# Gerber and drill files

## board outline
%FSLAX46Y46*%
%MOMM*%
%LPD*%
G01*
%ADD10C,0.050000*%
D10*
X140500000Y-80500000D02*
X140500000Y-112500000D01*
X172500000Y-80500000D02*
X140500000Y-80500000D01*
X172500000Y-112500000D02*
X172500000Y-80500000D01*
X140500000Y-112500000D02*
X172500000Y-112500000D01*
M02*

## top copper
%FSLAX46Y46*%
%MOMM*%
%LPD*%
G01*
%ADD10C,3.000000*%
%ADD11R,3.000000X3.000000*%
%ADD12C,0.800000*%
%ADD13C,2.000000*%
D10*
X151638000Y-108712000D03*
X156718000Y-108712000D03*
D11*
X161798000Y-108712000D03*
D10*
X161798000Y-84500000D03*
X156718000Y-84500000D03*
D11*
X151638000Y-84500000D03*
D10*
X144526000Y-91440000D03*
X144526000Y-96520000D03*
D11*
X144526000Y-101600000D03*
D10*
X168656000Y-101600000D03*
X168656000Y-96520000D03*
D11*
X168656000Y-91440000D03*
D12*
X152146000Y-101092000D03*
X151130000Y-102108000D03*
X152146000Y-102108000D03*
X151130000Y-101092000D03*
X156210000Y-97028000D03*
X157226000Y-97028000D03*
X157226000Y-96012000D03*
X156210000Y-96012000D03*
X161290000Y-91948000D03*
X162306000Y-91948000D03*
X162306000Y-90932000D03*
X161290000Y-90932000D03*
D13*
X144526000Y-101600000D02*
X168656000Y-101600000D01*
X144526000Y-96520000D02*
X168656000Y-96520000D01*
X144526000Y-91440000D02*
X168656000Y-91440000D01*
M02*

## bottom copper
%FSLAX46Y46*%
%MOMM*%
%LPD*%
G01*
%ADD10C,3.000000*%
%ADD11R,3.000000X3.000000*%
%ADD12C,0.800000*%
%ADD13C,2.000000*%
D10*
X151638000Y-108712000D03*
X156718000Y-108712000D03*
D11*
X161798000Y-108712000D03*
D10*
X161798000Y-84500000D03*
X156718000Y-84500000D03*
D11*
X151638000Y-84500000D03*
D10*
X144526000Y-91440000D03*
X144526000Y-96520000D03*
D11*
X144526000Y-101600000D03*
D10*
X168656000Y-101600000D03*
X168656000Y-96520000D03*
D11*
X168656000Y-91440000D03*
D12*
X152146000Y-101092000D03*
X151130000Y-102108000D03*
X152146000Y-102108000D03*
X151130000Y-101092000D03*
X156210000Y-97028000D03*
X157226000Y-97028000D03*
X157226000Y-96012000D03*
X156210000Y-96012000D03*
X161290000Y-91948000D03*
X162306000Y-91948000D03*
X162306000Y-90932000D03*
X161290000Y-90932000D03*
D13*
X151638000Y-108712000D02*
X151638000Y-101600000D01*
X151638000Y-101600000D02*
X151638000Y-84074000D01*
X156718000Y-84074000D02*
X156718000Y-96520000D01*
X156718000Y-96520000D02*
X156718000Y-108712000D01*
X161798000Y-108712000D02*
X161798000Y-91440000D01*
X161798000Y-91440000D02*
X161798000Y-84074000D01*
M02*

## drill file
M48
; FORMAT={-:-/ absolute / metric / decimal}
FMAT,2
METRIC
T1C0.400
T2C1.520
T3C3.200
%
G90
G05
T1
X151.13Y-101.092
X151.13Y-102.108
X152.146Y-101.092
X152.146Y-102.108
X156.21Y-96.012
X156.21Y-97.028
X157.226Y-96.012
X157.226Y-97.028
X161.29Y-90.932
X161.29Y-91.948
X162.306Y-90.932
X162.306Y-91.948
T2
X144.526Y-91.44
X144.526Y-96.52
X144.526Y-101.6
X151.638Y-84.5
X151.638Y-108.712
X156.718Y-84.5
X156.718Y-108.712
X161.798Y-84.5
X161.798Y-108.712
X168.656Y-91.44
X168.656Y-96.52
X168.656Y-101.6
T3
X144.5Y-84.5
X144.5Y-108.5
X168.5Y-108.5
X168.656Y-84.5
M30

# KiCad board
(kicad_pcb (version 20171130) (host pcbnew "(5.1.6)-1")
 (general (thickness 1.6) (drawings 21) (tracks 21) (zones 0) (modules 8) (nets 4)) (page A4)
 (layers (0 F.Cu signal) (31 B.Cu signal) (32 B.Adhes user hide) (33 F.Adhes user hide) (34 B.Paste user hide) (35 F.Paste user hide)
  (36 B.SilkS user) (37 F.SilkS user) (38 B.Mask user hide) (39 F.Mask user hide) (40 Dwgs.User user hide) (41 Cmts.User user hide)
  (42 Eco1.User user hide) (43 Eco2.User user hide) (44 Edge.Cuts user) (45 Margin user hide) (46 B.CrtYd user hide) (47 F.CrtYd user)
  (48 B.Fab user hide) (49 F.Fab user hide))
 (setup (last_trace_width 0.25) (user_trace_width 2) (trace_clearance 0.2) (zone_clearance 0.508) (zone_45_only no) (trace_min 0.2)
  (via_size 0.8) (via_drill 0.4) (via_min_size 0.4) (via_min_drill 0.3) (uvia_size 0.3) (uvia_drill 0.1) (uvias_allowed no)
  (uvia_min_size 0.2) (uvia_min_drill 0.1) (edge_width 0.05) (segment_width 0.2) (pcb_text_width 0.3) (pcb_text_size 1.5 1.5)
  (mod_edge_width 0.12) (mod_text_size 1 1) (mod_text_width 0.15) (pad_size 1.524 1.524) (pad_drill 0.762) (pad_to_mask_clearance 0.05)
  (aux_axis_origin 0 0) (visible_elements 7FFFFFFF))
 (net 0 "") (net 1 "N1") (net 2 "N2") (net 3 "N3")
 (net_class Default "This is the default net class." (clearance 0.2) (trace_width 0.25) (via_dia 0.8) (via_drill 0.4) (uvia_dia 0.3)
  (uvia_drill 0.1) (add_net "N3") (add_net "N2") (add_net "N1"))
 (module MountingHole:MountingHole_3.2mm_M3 (layer F.Cu) (at 168.5 108.5)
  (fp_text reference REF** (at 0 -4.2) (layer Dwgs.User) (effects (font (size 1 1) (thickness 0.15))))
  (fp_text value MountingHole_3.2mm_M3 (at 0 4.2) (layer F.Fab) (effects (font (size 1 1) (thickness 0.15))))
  (pad 1 np_thru_hole circle (at 0 0) (size 3.2 3.2) (drill 3.2) (layers *.Cu *.Mask)))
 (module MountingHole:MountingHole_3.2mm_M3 (layer F.Cu) (at 144.5 108.5)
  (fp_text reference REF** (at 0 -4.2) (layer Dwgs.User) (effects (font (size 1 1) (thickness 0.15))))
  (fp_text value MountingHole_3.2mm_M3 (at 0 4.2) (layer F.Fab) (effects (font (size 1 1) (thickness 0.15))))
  (pad 1 np_thru_hole circle (at 0 0) (size 3.2 3.2) (drill 3.2) (layers *.Cu *.Mask)))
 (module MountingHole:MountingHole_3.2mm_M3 (layer F.Cu) (at 144.5 84.5)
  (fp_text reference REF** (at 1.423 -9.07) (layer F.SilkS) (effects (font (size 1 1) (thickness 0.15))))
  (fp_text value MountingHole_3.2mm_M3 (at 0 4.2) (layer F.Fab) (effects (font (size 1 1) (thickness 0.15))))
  (pad 1 np_thru_hole circle (at 0 0) (size 3.2 3.2) (drill 3.2) (layers *.Cu *.Mask)))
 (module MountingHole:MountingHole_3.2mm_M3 (layer F.Cu) (at 168.656 84.5)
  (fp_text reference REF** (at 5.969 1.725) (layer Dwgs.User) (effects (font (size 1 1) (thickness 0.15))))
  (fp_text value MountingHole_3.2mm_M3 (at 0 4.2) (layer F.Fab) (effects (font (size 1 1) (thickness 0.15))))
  (pad 1 np_thru_hole circle (at 0 0) (size 3.2 3.2) (drill 3.2) (layers *.Cu *.Mask)))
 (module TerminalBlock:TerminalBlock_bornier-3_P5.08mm (layer F.Cu) (at 161.798 108.712 180)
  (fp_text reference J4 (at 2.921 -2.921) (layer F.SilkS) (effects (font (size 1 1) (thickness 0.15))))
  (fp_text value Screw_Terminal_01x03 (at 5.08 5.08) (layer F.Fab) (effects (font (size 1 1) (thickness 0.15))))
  (pad 3 thru_hole circle (at 10.16 0 180) (size 3 3) (drill 1.52) (layers *.Cu *.Mask) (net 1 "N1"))
  (pad 2 thru_hole circle (at 5.08 0 180) (size 3 3) (drill 1.52) (layers *.Cu *.Mask) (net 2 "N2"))
  (pad 1 thru_hole rect (at 0 0 180) (size 3 3) (drill 1.52) (layers *.Cu *.Mask) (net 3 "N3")))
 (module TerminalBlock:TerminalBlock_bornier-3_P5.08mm (layer F.Cu) (at 151.638 84.5)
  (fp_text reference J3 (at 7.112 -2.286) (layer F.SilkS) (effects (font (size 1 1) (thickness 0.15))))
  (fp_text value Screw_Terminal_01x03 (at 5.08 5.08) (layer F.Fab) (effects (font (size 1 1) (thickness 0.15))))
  (pad 3 thru_hole circle (at 10.16 0) (size 3 3) (drill 1.52) (layers *.Cu *.Mask) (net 3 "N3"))
  (pad 2 thru_hole circle (at 5.08 0) (size 3 3) (drill 1.52) (layers *.Cu *.Mask) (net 2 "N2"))
  (pad 1 thru_hole rect (at 0 0) (size 3 3) (drill 1.52) (layers *.Cu *.Mask) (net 1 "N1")))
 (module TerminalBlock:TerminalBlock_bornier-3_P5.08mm (layer F.Cu) (at 144.526 101.6 90)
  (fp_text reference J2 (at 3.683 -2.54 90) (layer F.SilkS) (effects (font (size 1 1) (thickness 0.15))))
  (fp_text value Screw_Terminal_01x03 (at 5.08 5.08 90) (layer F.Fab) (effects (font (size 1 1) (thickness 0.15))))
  (pad 3 thru_hole circle (at 10.16 0 90) (size 3 3) (drill 1.52) (layers *.Cu *.Mask) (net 3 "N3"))
  (pad 2 thru_hole circle (at 5.08 0 90) (size 3 3) (drill 1.52) (layers *.Cu *.Mask) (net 2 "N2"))
  (pad 1 thru_hole rect (at 0 0 90) (size 3 3) (drill 1.52) (layers *.Cu *.Mask) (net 1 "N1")))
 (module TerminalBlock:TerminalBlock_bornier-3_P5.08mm (layer F.Cu) (at 168.656 91.44 270)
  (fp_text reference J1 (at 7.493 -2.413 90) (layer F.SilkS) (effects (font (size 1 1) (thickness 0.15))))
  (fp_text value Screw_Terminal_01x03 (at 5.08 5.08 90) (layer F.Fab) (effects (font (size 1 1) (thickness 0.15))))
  (pad 3 thru_hole circle (at 10.16 0 270) (size 3 3) (drill 1.52) (layers *.Cu *.Mask) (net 1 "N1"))
  (pad 2 thru_hole circle (at 5.08 0 270) (size 3 3) (drill 1.52) (layers *.Cu *.Mask) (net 2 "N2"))
  (pad 1 thru_hole rect (at 0 0 270) (size 3 3) (drill 1.52) (layers *.Cu *.Mask) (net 3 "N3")))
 (gr_line (start 140.5 80.5) (end 140.5 112.5) (layer Edge.Cuts) (width 0.05))
 (gr_line (start 172.5 80.5) (end 140.5 80.5) (layer Edge.Cuts) (width 0.05))
 (gr_line (start 172.5 112.5) (end 172.5 80.5) (layer Edge.Cuts) (width 0.05))
 (gr_line (start 140.5 112.5) (end 172.5 112.5) (layer Edge.Cuts) (width 0.05))
 (via (at 152.146 101.092) (size 0.8) (drill 0.4) (layers F.Cu B.Cu) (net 1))
 (via (at 151.13 102.108) (size 0.8) (drill 0.4) (layers F.Cu B.Cu) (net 1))
 (via (at 152.146 102.108) (size 0.8) (drill 0.4) (layers F.Cu B.Cu) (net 1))
 (segment (start 144.526 101.6) (end 168.656 101.6) (width 2) (layer F.Cu) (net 1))
 (segment (start 151.638 108.712) (end 151.638 101.6) (width 2) (layer B.Cu) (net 1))
 (segment (start 151.638 101.6) (end 151.638 84.074) (width 2) (layer B.Cu) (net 1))
 (via (at 151.13 101.092) (size 0.8) (drill 0.4) (layers F.Cu B.Cu) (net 1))
 (via (at 156.21 97.028) (size 0.8) (drill 0.4) (layers F.Cu B.Cu) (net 2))
 (via (at 157.226 97.028) (size 0.8) (drill 0.4) (layers F.Cu B.Cu) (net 2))
 (via (at 157.226 96.012) (size 0.8) (drill 0.4) (layers F.Cu B.Cu) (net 2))
 (segment (start 144.526 96.52) (end 168.656 96.52) (width 2) (layer F.Cu) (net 2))
 (segment (start 156.718 84.074) (end 156.718 96.52) (width 2) (layer B.Cu) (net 2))
 (segment (start 156.718 96.52) (end 156.718 108.712) (width 2) (layer B.Cu) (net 2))
 (via (at 156.21 96.012) (size 0.8) (drill 0.4) (layers F.Cu B.Cu) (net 2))
 (via (at 161.29 91.948) (size 0.8) (drill 0.4) (layers F.Cu B.Cu) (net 3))
 (via (at 162.306 91.948) (size 0.8) (drill 0.4) (layers F.Cu B.Cu) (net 3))
 (via (at 162.306 90.932) (size 0.8) (drill 0.4) (layers F.Cu B.Cu) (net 3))
 (segment (start 144.526 91.44) (end 168.656 91.44) (width 2) (layer F.Cu) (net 3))
 (segment (start 161.798 108.712) (end 161.798 91.44) (width 2) (layer B.Cu) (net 3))
 (segment (start 161.798 91.44) (end 161.798 84.074) (width 2) (layer B.Cu) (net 3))
 (via (at 161.29 90.932) (size 0.8) (drill 0.4) (layers F.Cu B.Cu) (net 3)))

